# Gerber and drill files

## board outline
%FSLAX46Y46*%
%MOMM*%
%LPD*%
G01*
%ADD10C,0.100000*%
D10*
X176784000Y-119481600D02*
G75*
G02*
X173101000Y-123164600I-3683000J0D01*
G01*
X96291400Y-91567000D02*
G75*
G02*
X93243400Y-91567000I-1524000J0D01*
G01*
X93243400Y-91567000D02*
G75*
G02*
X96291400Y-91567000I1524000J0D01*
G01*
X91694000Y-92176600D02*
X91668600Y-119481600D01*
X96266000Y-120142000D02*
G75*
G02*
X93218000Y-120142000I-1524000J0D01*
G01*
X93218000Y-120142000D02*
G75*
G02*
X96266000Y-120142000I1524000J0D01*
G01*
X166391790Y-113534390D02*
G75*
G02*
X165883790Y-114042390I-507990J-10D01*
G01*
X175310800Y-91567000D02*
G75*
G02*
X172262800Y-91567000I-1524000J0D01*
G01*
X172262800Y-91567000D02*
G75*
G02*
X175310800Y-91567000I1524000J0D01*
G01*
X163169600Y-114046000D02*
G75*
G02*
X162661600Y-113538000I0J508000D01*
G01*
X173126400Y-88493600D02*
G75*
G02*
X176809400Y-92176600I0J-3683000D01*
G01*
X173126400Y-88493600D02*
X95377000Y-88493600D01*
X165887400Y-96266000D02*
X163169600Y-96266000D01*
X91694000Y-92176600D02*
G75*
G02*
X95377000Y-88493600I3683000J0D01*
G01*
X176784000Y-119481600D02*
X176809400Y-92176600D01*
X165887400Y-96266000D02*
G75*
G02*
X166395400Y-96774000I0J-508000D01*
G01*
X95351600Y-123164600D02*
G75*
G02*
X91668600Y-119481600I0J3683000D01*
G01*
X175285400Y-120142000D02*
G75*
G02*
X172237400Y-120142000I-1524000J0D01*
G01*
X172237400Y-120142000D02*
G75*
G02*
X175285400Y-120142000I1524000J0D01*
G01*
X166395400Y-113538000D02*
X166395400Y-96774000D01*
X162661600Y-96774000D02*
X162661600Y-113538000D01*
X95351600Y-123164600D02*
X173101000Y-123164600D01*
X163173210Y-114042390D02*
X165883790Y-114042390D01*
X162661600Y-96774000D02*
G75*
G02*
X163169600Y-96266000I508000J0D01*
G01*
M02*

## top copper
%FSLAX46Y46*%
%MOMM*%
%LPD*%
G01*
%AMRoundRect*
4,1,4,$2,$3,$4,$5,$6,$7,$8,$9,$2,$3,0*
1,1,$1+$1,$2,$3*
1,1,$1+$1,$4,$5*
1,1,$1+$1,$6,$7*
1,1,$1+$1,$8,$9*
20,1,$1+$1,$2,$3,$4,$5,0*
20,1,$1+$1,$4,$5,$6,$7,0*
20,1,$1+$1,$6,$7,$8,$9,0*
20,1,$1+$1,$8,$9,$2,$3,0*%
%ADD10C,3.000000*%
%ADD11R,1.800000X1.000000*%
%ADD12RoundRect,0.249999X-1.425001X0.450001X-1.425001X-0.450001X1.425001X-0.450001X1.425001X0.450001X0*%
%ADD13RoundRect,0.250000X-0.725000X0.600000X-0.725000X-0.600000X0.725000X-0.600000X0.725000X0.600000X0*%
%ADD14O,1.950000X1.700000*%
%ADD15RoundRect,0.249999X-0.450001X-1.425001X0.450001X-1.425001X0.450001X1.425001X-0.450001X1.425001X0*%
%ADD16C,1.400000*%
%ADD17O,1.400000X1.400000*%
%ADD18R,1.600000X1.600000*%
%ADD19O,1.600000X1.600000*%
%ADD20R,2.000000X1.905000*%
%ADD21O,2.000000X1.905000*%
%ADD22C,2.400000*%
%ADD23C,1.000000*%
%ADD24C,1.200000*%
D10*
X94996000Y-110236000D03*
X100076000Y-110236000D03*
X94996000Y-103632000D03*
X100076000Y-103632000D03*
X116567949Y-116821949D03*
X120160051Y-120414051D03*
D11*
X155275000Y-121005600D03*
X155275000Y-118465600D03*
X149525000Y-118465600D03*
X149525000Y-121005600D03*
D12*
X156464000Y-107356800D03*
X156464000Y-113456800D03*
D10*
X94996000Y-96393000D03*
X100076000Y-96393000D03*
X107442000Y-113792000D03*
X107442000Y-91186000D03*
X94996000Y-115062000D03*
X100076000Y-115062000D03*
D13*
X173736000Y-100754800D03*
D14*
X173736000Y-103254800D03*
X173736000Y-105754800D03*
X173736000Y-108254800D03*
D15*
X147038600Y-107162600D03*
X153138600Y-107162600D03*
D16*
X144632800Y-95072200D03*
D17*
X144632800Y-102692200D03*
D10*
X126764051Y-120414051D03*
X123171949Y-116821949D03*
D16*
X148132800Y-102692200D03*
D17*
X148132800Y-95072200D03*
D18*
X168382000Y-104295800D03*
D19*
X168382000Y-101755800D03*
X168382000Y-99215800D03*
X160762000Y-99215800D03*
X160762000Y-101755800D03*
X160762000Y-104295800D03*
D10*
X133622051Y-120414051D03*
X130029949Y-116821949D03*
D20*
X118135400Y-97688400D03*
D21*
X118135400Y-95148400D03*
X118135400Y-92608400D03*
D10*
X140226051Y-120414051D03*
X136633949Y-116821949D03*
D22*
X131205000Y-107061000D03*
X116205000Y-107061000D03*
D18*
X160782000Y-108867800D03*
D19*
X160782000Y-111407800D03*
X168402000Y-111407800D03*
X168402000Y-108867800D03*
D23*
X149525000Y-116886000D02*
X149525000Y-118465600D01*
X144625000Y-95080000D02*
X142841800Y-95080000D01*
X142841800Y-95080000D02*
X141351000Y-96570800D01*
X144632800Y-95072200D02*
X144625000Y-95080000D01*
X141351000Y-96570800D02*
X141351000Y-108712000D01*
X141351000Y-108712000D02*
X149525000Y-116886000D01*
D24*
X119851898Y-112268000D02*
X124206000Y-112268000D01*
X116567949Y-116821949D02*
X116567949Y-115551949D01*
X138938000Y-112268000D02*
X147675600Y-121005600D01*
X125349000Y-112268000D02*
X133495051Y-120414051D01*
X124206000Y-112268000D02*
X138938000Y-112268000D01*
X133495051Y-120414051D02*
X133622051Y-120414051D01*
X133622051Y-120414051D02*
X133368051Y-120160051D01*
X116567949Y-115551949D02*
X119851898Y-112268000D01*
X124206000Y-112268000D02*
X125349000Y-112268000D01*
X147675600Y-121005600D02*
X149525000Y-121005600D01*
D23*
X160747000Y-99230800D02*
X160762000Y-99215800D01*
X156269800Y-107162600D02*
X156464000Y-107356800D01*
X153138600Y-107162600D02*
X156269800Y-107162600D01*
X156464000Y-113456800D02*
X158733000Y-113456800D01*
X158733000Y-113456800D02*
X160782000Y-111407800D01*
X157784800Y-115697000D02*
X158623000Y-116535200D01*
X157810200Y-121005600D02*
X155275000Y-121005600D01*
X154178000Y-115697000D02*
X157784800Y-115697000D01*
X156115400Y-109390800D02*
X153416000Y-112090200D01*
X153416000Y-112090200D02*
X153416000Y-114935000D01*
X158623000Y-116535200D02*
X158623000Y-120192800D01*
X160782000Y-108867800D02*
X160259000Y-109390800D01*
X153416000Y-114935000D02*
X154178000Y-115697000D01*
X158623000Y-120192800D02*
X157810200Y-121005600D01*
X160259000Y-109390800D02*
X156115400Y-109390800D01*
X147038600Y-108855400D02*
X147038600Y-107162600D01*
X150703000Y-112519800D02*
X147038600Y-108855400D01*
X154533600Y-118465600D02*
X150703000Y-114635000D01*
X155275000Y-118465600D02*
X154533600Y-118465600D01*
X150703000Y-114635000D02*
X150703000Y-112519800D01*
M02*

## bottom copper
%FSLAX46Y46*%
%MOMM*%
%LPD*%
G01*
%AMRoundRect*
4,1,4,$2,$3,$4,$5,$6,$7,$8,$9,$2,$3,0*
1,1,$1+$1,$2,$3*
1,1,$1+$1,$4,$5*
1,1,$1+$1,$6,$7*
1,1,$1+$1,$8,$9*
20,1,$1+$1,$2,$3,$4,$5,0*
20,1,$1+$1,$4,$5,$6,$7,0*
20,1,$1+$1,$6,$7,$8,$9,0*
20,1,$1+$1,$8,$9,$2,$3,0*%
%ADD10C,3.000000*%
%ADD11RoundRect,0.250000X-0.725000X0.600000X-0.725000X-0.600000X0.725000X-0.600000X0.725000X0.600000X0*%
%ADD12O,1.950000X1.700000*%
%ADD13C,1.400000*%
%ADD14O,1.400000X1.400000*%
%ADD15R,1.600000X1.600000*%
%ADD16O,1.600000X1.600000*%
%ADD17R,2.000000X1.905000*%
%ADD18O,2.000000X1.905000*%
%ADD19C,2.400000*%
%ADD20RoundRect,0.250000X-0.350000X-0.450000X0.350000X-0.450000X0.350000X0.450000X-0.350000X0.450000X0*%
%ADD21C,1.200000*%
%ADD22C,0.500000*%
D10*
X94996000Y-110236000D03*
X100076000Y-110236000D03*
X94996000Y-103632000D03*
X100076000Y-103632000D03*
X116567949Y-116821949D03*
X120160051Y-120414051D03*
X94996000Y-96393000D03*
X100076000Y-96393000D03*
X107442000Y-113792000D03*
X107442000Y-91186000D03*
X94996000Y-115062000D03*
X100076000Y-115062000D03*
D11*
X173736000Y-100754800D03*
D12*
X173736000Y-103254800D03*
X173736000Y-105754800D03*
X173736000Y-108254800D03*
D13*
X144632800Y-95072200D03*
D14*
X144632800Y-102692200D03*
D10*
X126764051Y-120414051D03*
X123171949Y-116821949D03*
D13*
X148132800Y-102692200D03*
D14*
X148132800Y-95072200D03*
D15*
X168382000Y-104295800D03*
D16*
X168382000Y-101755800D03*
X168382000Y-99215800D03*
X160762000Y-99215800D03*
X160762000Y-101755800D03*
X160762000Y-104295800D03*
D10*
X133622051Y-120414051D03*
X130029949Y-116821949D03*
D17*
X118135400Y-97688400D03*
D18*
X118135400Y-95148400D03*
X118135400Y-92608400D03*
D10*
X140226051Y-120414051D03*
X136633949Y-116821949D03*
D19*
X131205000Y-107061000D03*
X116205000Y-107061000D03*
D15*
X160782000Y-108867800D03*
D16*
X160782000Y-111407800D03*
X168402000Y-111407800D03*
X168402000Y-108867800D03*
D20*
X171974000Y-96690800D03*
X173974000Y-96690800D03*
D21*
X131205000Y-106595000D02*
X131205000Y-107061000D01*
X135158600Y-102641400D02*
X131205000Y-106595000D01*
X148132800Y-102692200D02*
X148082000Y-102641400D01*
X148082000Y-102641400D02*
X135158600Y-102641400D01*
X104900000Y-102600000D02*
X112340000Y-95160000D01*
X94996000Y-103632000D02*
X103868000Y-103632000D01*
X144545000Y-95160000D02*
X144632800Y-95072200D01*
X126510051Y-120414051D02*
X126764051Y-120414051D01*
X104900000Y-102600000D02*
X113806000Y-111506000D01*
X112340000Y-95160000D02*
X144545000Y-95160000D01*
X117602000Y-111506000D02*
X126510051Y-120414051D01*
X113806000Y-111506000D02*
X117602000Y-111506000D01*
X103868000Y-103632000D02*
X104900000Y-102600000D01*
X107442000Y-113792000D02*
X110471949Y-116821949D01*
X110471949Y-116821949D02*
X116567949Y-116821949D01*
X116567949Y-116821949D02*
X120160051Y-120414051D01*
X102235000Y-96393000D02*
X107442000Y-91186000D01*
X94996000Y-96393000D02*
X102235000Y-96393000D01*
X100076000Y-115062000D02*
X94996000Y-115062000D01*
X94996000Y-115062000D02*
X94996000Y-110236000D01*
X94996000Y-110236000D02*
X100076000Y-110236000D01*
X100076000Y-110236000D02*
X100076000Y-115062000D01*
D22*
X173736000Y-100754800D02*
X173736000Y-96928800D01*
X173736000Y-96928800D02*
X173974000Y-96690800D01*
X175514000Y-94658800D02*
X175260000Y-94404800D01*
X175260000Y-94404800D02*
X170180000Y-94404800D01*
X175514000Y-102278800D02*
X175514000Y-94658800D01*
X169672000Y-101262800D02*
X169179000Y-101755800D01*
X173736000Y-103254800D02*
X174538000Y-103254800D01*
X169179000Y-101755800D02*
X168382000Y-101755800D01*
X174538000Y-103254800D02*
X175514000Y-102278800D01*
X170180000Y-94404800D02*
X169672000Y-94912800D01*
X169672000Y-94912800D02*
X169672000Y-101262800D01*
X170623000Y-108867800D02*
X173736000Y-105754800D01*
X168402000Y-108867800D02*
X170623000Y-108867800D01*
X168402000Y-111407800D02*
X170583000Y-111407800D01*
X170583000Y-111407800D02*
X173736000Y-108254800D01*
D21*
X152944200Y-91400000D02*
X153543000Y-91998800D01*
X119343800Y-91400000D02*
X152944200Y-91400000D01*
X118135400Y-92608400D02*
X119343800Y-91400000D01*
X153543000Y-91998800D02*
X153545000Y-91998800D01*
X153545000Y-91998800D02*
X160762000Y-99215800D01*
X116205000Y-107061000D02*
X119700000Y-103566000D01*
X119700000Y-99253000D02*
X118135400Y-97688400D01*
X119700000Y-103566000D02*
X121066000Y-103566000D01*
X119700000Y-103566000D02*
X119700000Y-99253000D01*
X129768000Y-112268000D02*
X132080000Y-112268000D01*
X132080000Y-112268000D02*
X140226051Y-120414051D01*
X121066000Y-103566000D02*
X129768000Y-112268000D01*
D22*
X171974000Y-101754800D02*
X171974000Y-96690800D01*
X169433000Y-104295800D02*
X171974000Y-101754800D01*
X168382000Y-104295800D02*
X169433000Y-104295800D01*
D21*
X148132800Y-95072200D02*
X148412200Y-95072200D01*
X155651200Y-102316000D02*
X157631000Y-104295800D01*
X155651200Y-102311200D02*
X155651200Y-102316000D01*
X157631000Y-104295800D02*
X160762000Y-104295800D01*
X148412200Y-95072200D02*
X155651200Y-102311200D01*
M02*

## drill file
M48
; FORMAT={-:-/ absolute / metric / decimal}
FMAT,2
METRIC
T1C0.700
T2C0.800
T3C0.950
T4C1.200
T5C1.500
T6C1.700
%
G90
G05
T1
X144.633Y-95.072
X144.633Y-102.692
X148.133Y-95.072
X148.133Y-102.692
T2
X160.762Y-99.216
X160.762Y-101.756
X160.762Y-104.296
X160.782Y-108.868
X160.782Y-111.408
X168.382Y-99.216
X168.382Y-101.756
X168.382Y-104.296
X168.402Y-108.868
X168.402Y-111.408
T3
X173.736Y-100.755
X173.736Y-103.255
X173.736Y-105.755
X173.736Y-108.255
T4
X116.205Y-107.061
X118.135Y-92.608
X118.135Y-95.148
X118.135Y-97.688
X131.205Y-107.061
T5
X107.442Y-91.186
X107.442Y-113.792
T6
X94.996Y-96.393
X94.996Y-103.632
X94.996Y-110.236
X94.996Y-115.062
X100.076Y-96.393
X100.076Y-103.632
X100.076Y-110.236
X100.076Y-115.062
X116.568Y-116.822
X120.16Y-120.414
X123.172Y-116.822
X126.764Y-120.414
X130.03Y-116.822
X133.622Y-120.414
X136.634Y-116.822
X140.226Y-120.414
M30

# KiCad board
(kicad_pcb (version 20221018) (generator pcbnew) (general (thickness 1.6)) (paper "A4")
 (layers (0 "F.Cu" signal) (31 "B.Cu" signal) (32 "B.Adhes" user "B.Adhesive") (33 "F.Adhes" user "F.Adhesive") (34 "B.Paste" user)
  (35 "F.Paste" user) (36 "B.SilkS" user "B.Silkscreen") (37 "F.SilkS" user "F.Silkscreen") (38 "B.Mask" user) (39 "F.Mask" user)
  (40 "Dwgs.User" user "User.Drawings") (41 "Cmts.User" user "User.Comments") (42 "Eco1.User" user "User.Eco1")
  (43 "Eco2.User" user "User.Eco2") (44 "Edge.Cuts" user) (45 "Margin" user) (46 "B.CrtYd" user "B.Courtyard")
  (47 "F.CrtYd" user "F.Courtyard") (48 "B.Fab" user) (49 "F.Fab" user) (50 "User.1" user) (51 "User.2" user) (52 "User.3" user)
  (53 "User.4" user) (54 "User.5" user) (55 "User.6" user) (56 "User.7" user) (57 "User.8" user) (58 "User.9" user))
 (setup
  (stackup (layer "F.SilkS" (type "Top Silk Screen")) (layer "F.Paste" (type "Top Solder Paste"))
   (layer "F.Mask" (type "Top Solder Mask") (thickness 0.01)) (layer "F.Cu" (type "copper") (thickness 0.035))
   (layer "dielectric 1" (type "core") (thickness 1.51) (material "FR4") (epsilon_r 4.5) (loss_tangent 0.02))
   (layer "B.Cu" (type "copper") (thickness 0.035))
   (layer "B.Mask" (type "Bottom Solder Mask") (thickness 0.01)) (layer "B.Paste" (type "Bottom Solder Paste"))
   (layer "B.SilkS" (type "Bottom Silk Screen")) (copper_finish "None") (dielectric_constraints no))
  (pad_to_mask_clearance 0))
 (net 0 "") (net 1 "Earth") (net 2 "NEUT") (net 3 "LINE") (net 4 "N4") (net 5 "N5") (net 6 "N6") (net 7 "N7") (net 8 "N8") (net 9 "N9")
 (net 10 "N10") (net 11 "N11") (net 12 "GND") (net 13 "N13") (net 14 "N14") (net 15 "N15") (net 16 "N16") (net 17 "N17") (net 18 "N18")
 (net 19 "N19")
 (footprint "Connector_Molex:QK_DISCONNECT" (layer "F.Cu") (at 97.536 110.236)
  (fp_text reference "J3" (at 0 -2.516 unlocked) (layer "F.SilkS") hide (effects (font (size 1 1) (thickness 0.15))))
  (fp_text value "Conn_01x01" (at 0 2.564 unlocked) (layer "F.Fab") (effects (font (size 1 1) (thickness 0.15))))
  (pad "1" thru_hole circle (at -2.54 0) (size 3 3) (drill 1.7) (layers "*.Cu" "*.Mask") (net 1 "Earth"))
  (pad "1" thru_hole circle (at 2.54 0) (size 3 3) (drill 1.7) (layers "*.Cu" "*.Mask") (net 1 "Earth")))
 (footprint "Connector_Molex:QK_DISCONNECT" (layer "F.Cu") (at 97.536 103.632)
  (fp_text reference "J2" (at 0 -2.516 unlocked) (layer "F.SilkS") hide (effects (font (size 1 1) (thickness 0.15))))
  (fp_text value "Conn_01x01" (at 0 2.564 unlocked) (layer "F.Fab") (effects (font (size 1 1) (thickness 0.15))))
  (pad "1" thru_hole circle (at -2.54 0) (size 3 3) (drill 1.7) (layers "*.Cu" "*.Mask") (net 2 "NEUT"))
  (pad "1" thru_hole circle (at 2.54 0) (size 3 3) (drill 1.7) (layers "*.Cu" "*.Mask") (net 2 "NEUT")))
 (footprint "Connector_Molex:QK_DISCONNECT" (layer "F.Cu") (at 118.364 118.618 -45)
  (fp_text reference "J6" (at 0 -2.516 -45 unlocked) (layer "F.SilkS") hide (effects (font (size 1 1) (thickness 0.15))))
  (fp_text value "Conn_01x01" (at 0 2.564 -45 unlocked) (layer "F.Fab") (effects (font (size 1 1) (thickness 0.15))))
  (pad "1" thru_hole circle (at -2.54 0 315) (size 3 3) (drill 1.7) (layers "*.Cu" "*.Mask") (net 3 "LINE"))
  (pad "1" thru_hole circle (at 2.54 0 315) (size 3 3) (drill 1.7) (layers "*.Cu" "*.Mask") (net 3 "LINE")))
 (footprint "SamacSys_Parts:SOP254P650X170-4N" (layer "F.Cu") (at 152.4 119.7356 180)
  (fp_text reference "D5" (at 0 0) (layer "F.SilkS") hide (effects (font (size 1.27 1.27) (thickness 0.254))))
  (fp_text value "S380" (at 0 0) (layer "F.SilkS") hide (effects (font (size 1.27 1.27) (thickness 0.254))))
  (pad "1" smd rect (at -2.875 -1.27 270) (size 1 1.8) (layers "F.Cu" "F.Paste" "F.Mask") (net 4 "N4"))
  (pad "2" smd rect (at -2.875 1.27 270) (size 1 1.8) (layers "F.Cu" "F.Paste" "F.Mask") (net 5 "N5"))
  (pad "3" smd rect (at 2.875 1.27 270) (size 1 1.8) (layers "F.Cu" "F.Paste" "F.Mask") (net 2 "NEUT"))
  (pad "4" smd rect (at 2.875 -1.27 270) (size 1 1.8) (layers "F.Cu" "F.Paste" "F.Mask") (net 3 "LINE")))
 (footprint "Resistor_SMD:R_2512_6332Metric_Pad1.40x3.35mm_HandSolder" (layer "F.Cu") (at 156.464 110.4068 -90)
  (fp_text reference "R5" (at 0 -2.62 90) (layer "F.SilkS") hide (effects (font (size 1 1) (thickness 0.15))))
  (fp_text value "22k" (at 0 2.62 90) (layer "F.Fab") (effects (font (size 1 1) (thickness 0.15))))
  (pad "1" smd roundrect (at -3.05 0 270) (size 1.4 3.35) (layers "F.Cu" "F.Paste" "F.Mask") (roundrect_rratio 0.178571) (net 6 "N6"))
  (pad "2" smd roundrect (at 3.05 0 270) (size 1.4 3.35) (layers "F.Cu" "F.Paste" "F.Mask") (roundrect_rratio 0.178571) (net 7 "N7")))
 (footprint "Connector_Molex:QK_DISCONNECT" (layer "F.Cu") (at 97.536 96.393)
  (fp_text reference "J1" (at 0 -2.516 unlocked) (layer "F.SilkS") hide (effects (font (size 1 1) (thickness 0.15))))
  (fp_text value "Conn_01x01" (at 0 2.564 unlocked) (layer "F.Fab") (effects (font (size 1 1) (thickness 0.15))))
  (pad "1" thru_hole circle (at -2.54 0) (size 3 3) (drill 1.7) (layers "*.Cu" "*.Mask") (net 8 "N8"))
  (pad "1" thru_hole circle (at 2.54 0) (size 3 3) (drill 1.7) (layers "*.Cu" "*.Mask") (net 8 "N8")))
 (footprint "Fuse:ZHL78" (layer "F.Cu") (at 107.442 102.489 90)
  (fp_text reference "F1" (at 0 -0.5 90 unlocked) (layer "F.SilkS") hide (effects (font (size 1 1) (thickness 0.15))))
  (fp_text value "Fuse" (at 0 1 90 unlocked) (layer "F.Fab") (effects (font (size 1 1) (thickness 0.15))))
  (pad "1" thru_hole circle (at -11.303 0 90) (size 3 3) (drill 1.5) (layers "*.Cu" "*.Mask") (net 3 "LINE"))
  (pad "2" thru_hole circle (at 11.303 0 90) (size 3 3) (drill 1.5) (layers "*.Cu" "*.Mask") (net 8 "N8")))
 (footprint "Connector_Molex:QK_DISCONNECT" (layer "F.Cu") (at 97.536 115.062)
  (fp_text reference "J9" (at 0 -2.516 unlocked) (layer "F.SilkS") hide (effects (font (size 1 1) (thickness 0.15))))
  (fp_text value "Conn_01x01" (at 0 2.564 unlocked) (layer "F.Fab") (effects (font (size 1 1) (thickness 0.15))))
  (pad "1" thru_hole circle (at -2.54 0) (size 3 3) (drill 1.7) (layers "*.Cu" "*.Mask") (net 1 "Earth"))
  (pad "1" thru_hole circle (at 2.54 0) (size 3 3) (drill 1.7) (layers "*.Cu" "*.Mask") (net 1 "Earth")))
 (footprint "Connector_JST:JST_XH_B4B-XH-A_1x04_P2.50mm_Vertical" (layer "F.Cu") (at 173.736 100.7548 -90)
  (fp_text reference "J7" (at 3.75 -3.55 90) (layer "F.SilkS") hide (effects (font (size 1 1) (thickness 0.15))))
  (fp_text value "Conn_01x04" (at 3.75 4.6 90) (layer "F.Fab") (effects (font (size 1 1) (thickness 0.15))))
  (pad "1" thru_hole roundrect (at 0 0 270) (size 1.7 1.95) (drill 0.95) (layers "*.Cu" "*.Mask") (roundrect_rratio 0.147059) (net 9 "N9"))
  (pad "2" thru_hole oval (at 2.5 0 270) (size 1.7 1.95) (drill 0.95) (layers "*.Cu" "*.Mask") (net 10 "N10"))
  (pad "3" thru_hole oval (at 5 0 270) (size 1.7 1.95) (drill 0.95) (layers "*.Cu" "*.Mask") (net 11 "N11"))
  (pad "4" thru_hole oval (at 7.5 0 270) (size 1.7 1.95) (drill 0.95) (layers "*.Cu" "*.Mask") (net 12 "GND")))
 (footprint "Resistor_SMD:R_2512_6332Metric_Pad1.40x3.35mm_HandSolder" (layer "F.Cu") (at 150.0886 107.1626)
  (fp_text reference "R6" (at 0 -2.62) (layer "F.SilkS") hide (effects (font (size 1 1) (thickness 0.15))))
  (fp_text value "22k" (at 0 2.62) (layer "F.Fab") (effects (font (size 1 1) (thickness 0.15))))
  (pad "1" smd roundrect (at -3.05 0) (size 1.4 3.35) (layers "F.Cu" "F.Paste" "F.Mask") (roundrect_rratio 0.178571) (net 5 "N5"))
  (pad "2" smd roundrect (at 3.05 0) (size 1.4 3.35) (layers "F.Cu" "F.Paste" "F.Mask") (roundrect_rratio 0.178571) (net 6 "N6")))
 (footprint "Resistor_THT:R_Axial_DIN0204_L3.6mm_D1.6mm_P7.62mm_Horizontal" (layer "F.Cu") (at 144.6328 95.0722 -90)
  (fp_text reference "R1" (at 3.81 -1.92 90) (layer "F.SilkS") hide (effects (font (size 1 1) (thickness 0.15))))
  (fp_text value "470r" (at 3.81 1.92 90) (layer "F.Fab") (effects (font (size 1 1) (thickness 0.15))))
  (pad "1" thru_hole circle (at 0 0 270) (size 1.4 1.4) (drill 0.7) (layers "*.Cu" "*.Mask") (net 2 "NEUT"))
  (pad "2" thru_hole oval (at 7.62 0 270) (size 1.4 1.4) (drill 0.7) (layers "*.Cu" "*.Mask") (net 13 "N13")))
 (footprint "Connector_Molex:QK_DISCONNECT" (layer "F.Cu") (at 124.968 118.618 135)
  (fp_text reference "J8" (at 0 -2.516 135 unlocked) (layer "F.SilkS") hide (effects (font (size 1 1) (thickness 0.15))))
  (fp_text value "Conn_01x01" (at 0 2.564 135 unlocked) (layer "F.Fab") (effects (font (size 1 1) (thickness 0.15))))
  (pad "1" thru_hole circle (at -2.54 0 135) (size 3 3) (drill 1.7) (layers "*.Cu" "*.Mask") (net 2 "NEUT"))
  (pad "1" thru_hole circle (at 2.54 0 135) (size 3 3) (drill 1.7) (layers "*.Cu" "*.Mask") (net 2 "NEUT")))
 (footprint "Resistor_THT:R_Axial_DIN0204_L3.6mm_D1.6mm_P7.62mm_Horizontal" (layer "F.Cu") (at 148.1328 102.6922 90)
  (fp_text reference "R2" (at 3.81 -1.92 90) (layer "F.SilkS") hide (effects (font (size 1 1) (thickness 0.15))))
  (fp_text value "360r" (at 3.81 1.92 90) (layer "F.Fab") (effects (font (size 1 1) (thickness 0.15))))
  (pad "1" thru_hole circle (at 0 0 90) (size 1.4 1.4) (drill 0.7) (layers "*.Cu" "*.Mask") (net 13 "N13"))
  (pad "2" thru_hole oval (at 7.62 0 90) (size 1.4 1.4) (drill 0.7) (layers "*.Cu" "*.Mask") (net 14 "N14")))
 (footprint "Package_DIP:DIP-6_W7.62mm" (layer "F.Cu") (at 168.382 104.2958 180)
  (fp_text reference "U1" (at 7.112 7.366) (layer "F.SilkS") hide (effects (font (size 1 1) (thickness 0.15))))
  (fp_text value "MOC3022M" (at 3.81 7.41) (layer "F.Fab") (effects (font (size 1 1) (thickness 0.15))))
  (pad "1" thru_hole rect (at 0 0 180) (size 1.6 1.6) (drill 0.8) (layers "*.Cu" "*.Mask") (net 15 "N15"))
  (pad "2" thru_hole oval (at 0 2.54 180) (size 1.6 1.6) (drill 0.8) (layers "*.Cu" "*.Mask") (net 10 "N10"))
  (pad "3" thru_hole oval (at 0 5.08 180) (size 1.6 1.6) (drill 0.8) (layers "*.Cu" "*.Mask") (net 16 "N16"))
  (pad "4" thru_hole oval (at 7.62 5.08 180) (size 1.6 1.6) (drill 0.8) (layers "*.Cu" "*.Mask") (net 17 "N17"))
  (pad "5" thru_hole oval (at 7.62 2.54 180) (size 1.6 1.6) (drill 0.8) (layers "*.Cu" "*.Mask") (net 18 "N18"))
  (pad "6" thru_hole oval (at 7.62 0 180) (size 1.6 1.6) (drill 0.8) (layers "*.Cu" "*.Mask") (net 14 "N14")))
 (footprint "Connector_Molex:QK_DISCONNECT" (layer "F.Cu") (at 131.826 118.618 135)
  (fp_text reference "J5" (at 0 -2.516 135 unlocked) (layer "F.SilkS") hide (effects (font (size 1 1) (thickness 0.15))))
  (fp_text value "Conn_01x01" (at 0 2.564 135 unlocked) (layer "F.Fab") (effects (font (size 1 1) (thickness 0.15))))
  (pad "1" thru_hole circle (at -2.54 0 135) (size 3 3) (drill 1.7) (layers "*.Cu" "*.Mask") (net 3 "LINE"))
  (pad "1" thru_hole circle (at 2.54 0 135) (size 3 3) (drill 1.7) (layers "*.Cu" "*.Mask") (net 3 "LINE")))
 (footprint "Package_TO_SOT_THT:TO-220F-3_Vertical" (layer "F.Cu") (at 118.1354 97.6884 90)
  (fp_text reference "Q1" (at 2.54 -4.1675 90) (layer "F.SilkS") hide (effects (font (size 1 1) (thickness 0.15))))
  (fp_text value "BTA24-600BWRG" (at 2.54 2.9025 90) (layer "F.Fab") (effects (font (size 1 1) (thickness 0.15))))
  (pad "1" thru_hole rect (at 0 0 90) (size 1.905 2) (drill 1.2) (layers "*.Cu" "*.Mask") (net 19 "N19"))
  (pad "2" thru_hole oval (at 2.54 0 90) (size 1.905 2) (drill 1.2) (layers "*.Cu" "*.Mask") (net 2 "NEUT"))
  (pad "3" thru_hole oval (at 5.08 0 90) (size 1.905 2) (drill 1.2) (layers "*.Cu" "*.Mask") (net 17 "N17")))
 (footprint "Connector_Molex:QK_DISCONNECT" (layer "F.Cu") (at 138.43 118.618 135)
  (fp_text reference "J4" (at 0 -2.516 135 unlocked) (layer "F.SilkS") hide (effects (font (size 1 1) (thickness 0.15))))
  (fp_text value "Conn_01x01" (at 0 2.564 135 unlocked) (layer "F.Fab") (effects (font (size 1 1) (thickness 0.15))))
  (pad "1" thru_hole circle (at -2.54 0 135) (size 3 3) (drill 1.7) (layers "*.Cu" "*.Mask") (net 19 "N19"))
  (pad "1" thru_hole circle (at 2.54 0 135) (size 3 3) (drill 1.7) (layers "*.Cu" "*.Mask") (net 19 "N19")))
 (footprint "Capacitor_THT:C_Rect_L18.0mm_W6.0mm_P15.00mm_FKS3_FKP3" (layer "F.Cu") (at 131.205 107.061 180)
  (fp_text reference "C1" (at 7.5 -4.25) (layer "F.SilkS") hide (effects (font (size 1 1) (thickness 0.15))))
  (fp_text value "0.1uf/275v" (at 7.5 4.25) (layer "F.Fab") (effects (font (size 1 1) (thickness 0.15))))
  (pad "1" thru_hole circle (at 0 0 180) (size 2.4 2.4) (drill 1.2) (layers "*.Cu" "*.Mask") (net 13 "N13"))
  (pad "2" thru_hole circle (at 15 0 180) (size 2.4 2.4) (drill 1.2) (layers "*.Cu" "*.Mask") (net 19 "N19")))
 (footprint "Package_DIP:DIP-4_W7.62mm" (layer "F.Cu") (at 160.782 108.8678)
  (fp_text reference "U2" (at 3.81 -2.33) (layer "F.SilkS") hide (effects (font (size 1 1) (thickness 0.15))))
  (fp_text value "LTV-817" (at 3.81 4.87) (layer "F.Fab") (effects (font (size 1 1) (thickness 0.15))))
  (pad "1" thru_hole rect (at 0 0) (size 1.6 1.6) (drill 0.8) (layers "*.Cu" "*.Mask") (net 4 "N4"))
  (pad "2" thru_hole oval (at 0 2.54) (size 1.6 1.6) (drill 0.8) (layers "*.Cu" "*.Mask") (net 7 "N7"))
  (pad "3" thru_hole oval (at 7.62 2.54) (size 1.6 1.6) (drill 0.8) (layers "*.Cu" "*.Mask") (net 12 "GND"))
  (pad "4" thru_hole oval (at 7.62 0) (size 1.6 1.6) (drill 0.8) (layers "*.Cu" "*.Mask") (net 11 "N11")))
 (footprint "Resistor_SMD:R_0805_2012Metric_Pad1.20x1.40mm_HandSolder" (layer "B.Cu") (at 172.974 96.6908)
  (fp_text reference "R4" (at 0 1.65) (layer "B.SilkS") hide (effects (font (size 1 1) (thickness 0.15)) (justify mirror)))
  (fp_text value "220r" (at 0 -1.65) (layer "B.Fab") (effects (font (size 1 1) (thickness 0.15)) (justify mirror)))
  (pad "1" smd roundrect (at -1 0) (size 1.2 1.4) (layers "B.Cu" "B.Paste" "B.Mask") (roundrect_rratio 0.208333) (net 15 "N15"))
  (pad "2" smd roundrect (at 1 0) (size 1.2 1.4) (layers "B.Cu" "B.Paste" "B.Mask") (roundrect_rratio 0.208333) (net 9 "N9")))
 (gr_arc (start 176.784 119.4816) (mid 175.705274 122.085874) (end 173.101 123.1646) (stroke (width 0.1) (type default)) (layer "Edge.Cuts"))
 (gr_circle (center 94.7674 91.567) (end 96.2914 91.567) (stroke (width 0.1) (type default)) (fill none) (layer "Edge.Cuts"))
 (gr_line (start 91.694 92.1766) (end 91.6686 119.4816) (stroke (width 0.1) (type default)) (layer "Edge.Cuts"))
 (gr_circle (center 94.742 120.142) (end 96.266 120.142) (stroke (width 0.1) (type default)) (fill none) (layer "Edge.Cuts"))
 (gr_arc (start 166.39179 113.53439) (mid 166.243 113.8936) (end 165.88379 114.04239) (stroke (width 0.1) (type default))
  (layer "Edge.Cuts"))
 (gr_circle (center 173.7868 91.567) (end 175.3108 91.567) (stroke (width 0.1) (type default)) (fill none) (layer "Edge.Cuts"))
 (gr_arc (start 163.1696 114.046) (mid 162.81039 113.89721) (end 162.6616 113.538) (stroke (width 0.1) (type default)) (layer "Edge.Cuts"))
 (gr_arc (start 173.1264 88.4936) (mid 175.730674 89.572326) (end 176.8094 92.1766) (stroke (width 0.1) (type default)) (layer "Edge.Cuts"))
 (gr_line (start 173.1264 88.4936) (end 95.377 88.4936) (stroke (width 0.1) (type default)) (layer "Edge.Cuts"))
 (gr_line (start 165.8874 96.266) (end 163.1696 96.266) (stroke (width 0.1) (type default)) (layer "Edge.Cuts"))
 (gr_arc (start 91.694 92.1766) (mid 92.772726 89.572326) (end 95.377 88.4936) (stroke (width 0.1) (type default)) (layer "Edge.Cuts"))
 (gr_line (start 176.784 119.4816) (end 176.8094 92.1766) (stroke (width 0.1) (type default)) (layer "Edge.Cuts"))
 (gr_arc (start 165.8874 96.266) (mid 166.24661 96.41479) (end 166.3954 96.774) (stroke (width 0.1) (type default)) (layer "Edge.Cuts"))
 (gr_arc (start 95.3516 123.1646) (mid 92.747326 122.085874) (end 91.6686 119.4816) (stroke (width 0.1) (type default)) (layer "Edge.Cuts"))
 (gr_circle (center 173.7614 120.142) (end 175.2854 120.142) (stroke (width 0.1) (type default)) (fill none) (layer "Edge.Cuts"))
 (gr_line (start 166.3954 113.538) (end 166.3954 96.774) (stroke (width 0.1) (type default)) (layer "Edge.Cuts"))
 (gr_line (start 162.6616 96.774) (end 162.6616 113.538) (stroke (width 0.1) (type default)) (layer "Edge.Cuts"))
 (gr_line (start 95.3516 123.1646) (end 173.101 123.1646) (stroke (width 0.1) (type default)) (layer "Edge.Cuts"))
 (gr_line (start 163.17321 114.04239) (end 165.88379 114.04239) (stroke (width 0.1) (type default)) (layer "Edge.Cuts"))
 (gr_arc (start 162.6616 96.774) (mid 162.81039 96.41479) (end 163.1696 96.266) (stroke (width 0.1) (type default)) (layer "Edge.Cuts"))
 (segment (start 131.205 106.595) (end 131.205 107.061) (width 1.2) (layer "B.Cu") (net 13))
 (segment (start 135.1586 102.6414) (end 131.205 106.595) (width 1.2) (layer "B.Cu") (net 13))
 (segment (start 148.1328 102.6922) (end 148.082 102.6414) (width 1.2) (layer "B.Cu") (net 13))
 (segment (start 148.082 102.6414) (end 135.1586 102.6414) (width 1.2) (layer "B.Cu") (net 13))
 (segment (start 149.525 116.886) (end 149.525 118.4656) (width 1) (layer "F.Cu") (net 2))
 (segment (start 144.625 95.08) (end 142.8418 95.08) (width 1) (layer "F.Cu") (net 2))
 (segment (start 142.8418 95.08) (end 141.351 96.5708) (width 1) (layer "F.Cu") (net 2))
 (segment (start 144.6328 95.0722) (end 144.625 95.08) (width 1) (layer "F.Cu") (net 2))
 (segment (start 141.351 96.5708) (end 141.351 108.712) (width 1) (layer "F.Cu") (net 2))
 (segment (start 141.351 108.712) (end 149.525 116.886) (width 1) (layer "F.Cu") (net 2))
 (segment (start 104.9 102.6) (end 112.34 95.16) (width 1.2) (layer "B.Cu") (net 2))
 (segment (start 94.996 103.632) (end 103.868 103.632) (width 1.2) (layer "B.Cu") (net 2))
 (segment (start 144.545 95.16) (end 144.6328 95.0722) (width 1.2) (layer "B.Cu") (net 2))
 (segment (start 126.510051 120.414051) (end 126.764051 120.414051) (width 1.2) (layer "B.Cu") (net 2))
 (segment (start 104.9 102.6) (end 113.806 111.506) (width 1.2) (layer "B.Cu") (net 2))
 (segment (start 112.34 95.16) (end 144.545 95.16) (width 1.2) (layer "B.Cu") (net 2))
 (segment (start 117.602 111.506) (end 126.510051 120.414051) (width 1.2) (layer "B.Cu") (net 2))
 (segment (start 113.806 111.506) (end 117.602 111.506) (width 1.2) (layer "B.Cu") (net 2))
 (segment (start 103.868 103.632) (end 104.9 102.6) (width 1.2) (layer "B.Cu") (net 2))
 (segment (start 119.851898 112.268) (end 124.206 112.268) (width 1.2) (layer "F.Cu") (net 3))
 (segment (start 116.567949 116.821949) (end 116.567949 115.551949) (width 1.2) (layer "F.Cu") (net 3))
 (segment (start 138.938 112.268) (end 147.6756 121.0056) (width 1.2) (layer "F.Cu") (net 3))
 (segment (start 125.349 112.268) (end 133.495051 120.414051) (width 1.2) (layer "F.Cu") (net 3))
 (segment (start 124.206 112.268) (end 138.938 112.268) (width 1.2) (layer "F.Cu") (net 3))
 (segment (start 133.495051 120.414051) (end 133.622051 120.414051) (width 1.2) (layer "F.Cu") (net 3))
 (segment (start 133.622051 120.414051) (end 133.368051 120.160051) (width 1.2) (layer "F.Cu") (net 3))
 (segment (start 116.567949 115.551949) (end 119.851898 112.268) (width 1.2) (layer "F.Cu") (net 3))
 (segment (start 124.206 112.268) (end 125.349 112.268) (width 1.2) (layer "F.Cu") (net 3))
 (segment (start 147.6756 121.0056) (end 149.525 121.0056) (width 1.2) (layer "F.Cu") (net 3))
 (segment (start 107.442 113.792) (end 110.471949 116.821949) (width 1.2) (layer "B.Cu") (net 3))
 (segment (start 110.471949 116.821949) (end 116.567949 116.821949) (width 1.2) (layer "B.Cu") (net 3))
 (segment (start 116.567949 116.821949) (end 120.160051 120.414051) (width 1.2) (layer "B.Cu") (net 3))
 (segment (start 102.235 96.393) (end 107.442 91.186) (width 1.2) (layer "B.Cu") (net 8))
 (segment (start 94.996 96.393) (end 102.235 96.393) (width 1.2) (layer "B.Cu") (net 8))
 (segment (start 100.076 115.062) (end 94.996 115.062) (width 1.2) (layer "B.Cu") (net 1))
 (segment (start 94.996 115.062) (end 94.996 110.236) (width 1.2) (layer "B.Cu") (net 1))
 (segment (start 94.996 110.236) (end 100.076 110.236) (width 1.2) (layer "B.Cu") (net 1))
 (segment (start 100.076 110.236) (end 100.076 115.062) (width 1.2) (layer "B.Cu") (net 1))
 (segment (start 173.736 100.7548) (end 173.736 96.9288) (width 0.5) (layer "B.Cu") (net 9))
 (segment (start 173.736 96.9288) (end 173.974 96.6908) (width 0.5) (layer "B.Cu") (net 9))
 (segment (start 175.514 94.6588) (end 175.26 94.4048) (width 0.5) (layer "B.Cu") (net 10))
 (segment (start 175.26 94.4048) (end 170.18 94.4048) (width 0.5) (layer "B.Cu") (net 10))
 (segment (start 175.514 102.2788) (end 175.514 94.6588) (width 0.5) (layer "B.Cu") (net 10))
 (segment (start 169.672 101.2628) (end 169.179 101.7558) (width 0.5) (layer "B.Cu") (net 10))
 (segment (start 173.736 103.2548) (end 174.538 103.2548) (width 0.5) (layer "B.Cu") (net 10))
 (segment (start 169.179 101.7558) (end 168.382 101.7558) (width 0.5) (layer "B.Cu") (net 10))
 (segment (start 174.538 103.2548) (end 175.514 102.2788) (width 0.5) (layer "B.Cu") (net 10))
 (segment (start 170.18 94.4048) (end 169.672 94.9128) (width 0.5) (layer "B.Cu") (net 10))
 (segment (start 169.672 94.9128) (end 169.672 101.2628) (width 0.5) (layer "B.Cu") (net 10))
 (segment (start 170.623 108.8678) (end 173.736 105.7548) (width 0.5) (layer "B.Cu") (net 11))
 (segment (start 168.402 108.8678) (end 170.623 108.8678) (width 0.5) (layer "B.Cu") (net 11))
 (segment (start 168.402 111.4078) (end 170.583 111.4078) (width 0.5) (layer "B.Cu") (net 12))
 (segment (start 170.583 111.4078) (end 173.736 108.2548) (width 0.5) (layer "B.Cu") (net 12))
 (segment (start 160.747 99.2308) (end 160.762 99.2158) (width 1) (layer "F.Cu") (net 17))
 (segment (start 152.9442 91.4) (end 153.543 91.9988) (width 1.2) (layer "B.Cu") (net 17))
 (segment (start 119.3438 91.4) (end 152.9442 91.4) (width 1.2) (layer "B.Cu") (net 17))
 (segment (start 118.1354 92.6084) (end 119.3438 91.4) (width 1.2) (layer "B.Cu") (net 17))
 (segment (start 153.543 91.9988) (end 153.545 91.9988) (width 1.2) (layer "B.Cu") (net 17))
 (segment (start 153.545 91.9988) (end 160.762 99.2158) (width 1.2) (layer "B.Cu") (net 17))
 (segment (start 116.205 107.061) (end 119.7 103.566) (width 1.2) (layer "B.Cu") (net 19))
 (segment (start 119.7 99.253) (end 118.1354 97.6884) (width 1.2) (layer "B.Cu") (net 19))
 (segment (start 119.7 103.566) (end 121.066 103.566) (width 1.2) (layer "B.Cu") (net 19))
 (segment (start 119.7 103.566) (end 119.7 99.253) (width 1.2) (layer "B.Cu") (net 19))
 (segment (start 129.768 112.268) (end 132.08 112.268) (width 1.2) (layer "B.Cu") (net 19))
 (segment (start 132.08 112.268) (end 140.226051 120.414051) (width 1.2) (layer "B.Cu") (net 19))
 (segment (start 121.066 103.566) (end 129.768 112.268) (width 1.2) (layer "B.Cu") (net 19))
 (segment (start 171.974 101.7548) (end 171.974 96.6908) (width 0.5) (layer "B.Cu") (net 15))
 (segment (start 169.433 104.2958) (end 171.974 101.7548) (width 0.5) (layer "B.Cu") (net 15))
 (segment (start 168.382 104.2958) (end 169.433 104.2958) (width 0.5) (layer "B.Cu") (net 15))
 (segment (start 156.2698 107.1626) (end 156.464 107.3568) (width 1) (layer "F.Cu") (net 6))
 (segment (start 153.1386 107.1626) (end 156.2698 107.1626) (width 1) (layer "F.Cu") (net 6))
 (segment (start 156.464 113.4568) (end 158.733 113.4568) (width 1) (layer "F.Cu") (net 7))
 (segment (start 158.733 113.4568) (end 160.782 111.4078) (width 1) (layer "F.Cu") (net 7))
 (segment (start 157.7848 115.697) (end 158.623 116.5352) (width 1) (layer "F.Cu") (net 4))
 (segment (start 157.8102 121.0056) (end 155.275 121.0056) (width 1) (layer "F.Cu") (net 4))
 (segment (start 154.178 115.697) (end 157.7848 115.697) (width 1) (layer "F.Cu") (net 4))
 (segment (start 156.1154 109.3908) (end 153.416 112.0902) (width 1) (layer "F.Cu") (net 4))
 (segment (start 153.416 112.0902) (end 153.416 114.935) (width 1) (layer "F.Cu") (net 4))
 (segment (start 158.623 116.5352) (end 158.623 120.1928) (width 1) (layer "F.Cu") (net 4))
 (segment (start 160.782 108.8678) (end 160.259 109.3908) (width 1) (layer "F.Cu") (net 4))
 (segment (start 153.416 114.935) (end 154.178 115.697) (width 1) (layer "F.Cu") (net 4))
 (segment (start 158.623 120.1928) (end 157.8102 121.0056) (width 1) (layer "F.Cu") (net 4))
 (segment (start 160.259 109.3908) (end 156.1154 109.3908) (width 1) (layer "F.Cu") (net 4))
 (segment (start 147.0386 108.8554) (end 147.0386 107.1626) (width 1) (layer "F.Cu") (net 5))
 (segment (start 150.703 112.5198) (end 147.0386 108.8554) (width 1) (layer "F.Cu") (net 5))
 (segment (start 154.5336 118.4656) (end 150.703 114.635) (width 1) (layer "F.Cu") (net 5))
 (segment (start 155.275 118.4656) (end 154.5336 118.4656) (width 1) (layer "F.Cu") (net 5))
 (segment (start 150.703 114.635) (end 150.703 112.5198) (width 1) (layer "F.Cu") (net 5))
 (segment (start 148.1328 95.0722) (end 148.4122 95.0722) (width 1.2) (layer "B.Cu") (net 14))
 (segment (start 155.6512 102.316) (end 157.631 104.2958) (width 1.2) (layer "B.Cu") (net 14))
 (segment (start 155.6512 102.3112) (end 155.6512 102.316) (width 1.2) (layer "B.Cu") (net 14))
 (segment (start 157.631 104.2958) (end 160.762 104.2958) (width 1.2) (layer "B.Cu") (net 14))
 (segment (start 148.4122 95.0722) (end 155.6512 102.3112) (width 1.2) (layer "B.Cu") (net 14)))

